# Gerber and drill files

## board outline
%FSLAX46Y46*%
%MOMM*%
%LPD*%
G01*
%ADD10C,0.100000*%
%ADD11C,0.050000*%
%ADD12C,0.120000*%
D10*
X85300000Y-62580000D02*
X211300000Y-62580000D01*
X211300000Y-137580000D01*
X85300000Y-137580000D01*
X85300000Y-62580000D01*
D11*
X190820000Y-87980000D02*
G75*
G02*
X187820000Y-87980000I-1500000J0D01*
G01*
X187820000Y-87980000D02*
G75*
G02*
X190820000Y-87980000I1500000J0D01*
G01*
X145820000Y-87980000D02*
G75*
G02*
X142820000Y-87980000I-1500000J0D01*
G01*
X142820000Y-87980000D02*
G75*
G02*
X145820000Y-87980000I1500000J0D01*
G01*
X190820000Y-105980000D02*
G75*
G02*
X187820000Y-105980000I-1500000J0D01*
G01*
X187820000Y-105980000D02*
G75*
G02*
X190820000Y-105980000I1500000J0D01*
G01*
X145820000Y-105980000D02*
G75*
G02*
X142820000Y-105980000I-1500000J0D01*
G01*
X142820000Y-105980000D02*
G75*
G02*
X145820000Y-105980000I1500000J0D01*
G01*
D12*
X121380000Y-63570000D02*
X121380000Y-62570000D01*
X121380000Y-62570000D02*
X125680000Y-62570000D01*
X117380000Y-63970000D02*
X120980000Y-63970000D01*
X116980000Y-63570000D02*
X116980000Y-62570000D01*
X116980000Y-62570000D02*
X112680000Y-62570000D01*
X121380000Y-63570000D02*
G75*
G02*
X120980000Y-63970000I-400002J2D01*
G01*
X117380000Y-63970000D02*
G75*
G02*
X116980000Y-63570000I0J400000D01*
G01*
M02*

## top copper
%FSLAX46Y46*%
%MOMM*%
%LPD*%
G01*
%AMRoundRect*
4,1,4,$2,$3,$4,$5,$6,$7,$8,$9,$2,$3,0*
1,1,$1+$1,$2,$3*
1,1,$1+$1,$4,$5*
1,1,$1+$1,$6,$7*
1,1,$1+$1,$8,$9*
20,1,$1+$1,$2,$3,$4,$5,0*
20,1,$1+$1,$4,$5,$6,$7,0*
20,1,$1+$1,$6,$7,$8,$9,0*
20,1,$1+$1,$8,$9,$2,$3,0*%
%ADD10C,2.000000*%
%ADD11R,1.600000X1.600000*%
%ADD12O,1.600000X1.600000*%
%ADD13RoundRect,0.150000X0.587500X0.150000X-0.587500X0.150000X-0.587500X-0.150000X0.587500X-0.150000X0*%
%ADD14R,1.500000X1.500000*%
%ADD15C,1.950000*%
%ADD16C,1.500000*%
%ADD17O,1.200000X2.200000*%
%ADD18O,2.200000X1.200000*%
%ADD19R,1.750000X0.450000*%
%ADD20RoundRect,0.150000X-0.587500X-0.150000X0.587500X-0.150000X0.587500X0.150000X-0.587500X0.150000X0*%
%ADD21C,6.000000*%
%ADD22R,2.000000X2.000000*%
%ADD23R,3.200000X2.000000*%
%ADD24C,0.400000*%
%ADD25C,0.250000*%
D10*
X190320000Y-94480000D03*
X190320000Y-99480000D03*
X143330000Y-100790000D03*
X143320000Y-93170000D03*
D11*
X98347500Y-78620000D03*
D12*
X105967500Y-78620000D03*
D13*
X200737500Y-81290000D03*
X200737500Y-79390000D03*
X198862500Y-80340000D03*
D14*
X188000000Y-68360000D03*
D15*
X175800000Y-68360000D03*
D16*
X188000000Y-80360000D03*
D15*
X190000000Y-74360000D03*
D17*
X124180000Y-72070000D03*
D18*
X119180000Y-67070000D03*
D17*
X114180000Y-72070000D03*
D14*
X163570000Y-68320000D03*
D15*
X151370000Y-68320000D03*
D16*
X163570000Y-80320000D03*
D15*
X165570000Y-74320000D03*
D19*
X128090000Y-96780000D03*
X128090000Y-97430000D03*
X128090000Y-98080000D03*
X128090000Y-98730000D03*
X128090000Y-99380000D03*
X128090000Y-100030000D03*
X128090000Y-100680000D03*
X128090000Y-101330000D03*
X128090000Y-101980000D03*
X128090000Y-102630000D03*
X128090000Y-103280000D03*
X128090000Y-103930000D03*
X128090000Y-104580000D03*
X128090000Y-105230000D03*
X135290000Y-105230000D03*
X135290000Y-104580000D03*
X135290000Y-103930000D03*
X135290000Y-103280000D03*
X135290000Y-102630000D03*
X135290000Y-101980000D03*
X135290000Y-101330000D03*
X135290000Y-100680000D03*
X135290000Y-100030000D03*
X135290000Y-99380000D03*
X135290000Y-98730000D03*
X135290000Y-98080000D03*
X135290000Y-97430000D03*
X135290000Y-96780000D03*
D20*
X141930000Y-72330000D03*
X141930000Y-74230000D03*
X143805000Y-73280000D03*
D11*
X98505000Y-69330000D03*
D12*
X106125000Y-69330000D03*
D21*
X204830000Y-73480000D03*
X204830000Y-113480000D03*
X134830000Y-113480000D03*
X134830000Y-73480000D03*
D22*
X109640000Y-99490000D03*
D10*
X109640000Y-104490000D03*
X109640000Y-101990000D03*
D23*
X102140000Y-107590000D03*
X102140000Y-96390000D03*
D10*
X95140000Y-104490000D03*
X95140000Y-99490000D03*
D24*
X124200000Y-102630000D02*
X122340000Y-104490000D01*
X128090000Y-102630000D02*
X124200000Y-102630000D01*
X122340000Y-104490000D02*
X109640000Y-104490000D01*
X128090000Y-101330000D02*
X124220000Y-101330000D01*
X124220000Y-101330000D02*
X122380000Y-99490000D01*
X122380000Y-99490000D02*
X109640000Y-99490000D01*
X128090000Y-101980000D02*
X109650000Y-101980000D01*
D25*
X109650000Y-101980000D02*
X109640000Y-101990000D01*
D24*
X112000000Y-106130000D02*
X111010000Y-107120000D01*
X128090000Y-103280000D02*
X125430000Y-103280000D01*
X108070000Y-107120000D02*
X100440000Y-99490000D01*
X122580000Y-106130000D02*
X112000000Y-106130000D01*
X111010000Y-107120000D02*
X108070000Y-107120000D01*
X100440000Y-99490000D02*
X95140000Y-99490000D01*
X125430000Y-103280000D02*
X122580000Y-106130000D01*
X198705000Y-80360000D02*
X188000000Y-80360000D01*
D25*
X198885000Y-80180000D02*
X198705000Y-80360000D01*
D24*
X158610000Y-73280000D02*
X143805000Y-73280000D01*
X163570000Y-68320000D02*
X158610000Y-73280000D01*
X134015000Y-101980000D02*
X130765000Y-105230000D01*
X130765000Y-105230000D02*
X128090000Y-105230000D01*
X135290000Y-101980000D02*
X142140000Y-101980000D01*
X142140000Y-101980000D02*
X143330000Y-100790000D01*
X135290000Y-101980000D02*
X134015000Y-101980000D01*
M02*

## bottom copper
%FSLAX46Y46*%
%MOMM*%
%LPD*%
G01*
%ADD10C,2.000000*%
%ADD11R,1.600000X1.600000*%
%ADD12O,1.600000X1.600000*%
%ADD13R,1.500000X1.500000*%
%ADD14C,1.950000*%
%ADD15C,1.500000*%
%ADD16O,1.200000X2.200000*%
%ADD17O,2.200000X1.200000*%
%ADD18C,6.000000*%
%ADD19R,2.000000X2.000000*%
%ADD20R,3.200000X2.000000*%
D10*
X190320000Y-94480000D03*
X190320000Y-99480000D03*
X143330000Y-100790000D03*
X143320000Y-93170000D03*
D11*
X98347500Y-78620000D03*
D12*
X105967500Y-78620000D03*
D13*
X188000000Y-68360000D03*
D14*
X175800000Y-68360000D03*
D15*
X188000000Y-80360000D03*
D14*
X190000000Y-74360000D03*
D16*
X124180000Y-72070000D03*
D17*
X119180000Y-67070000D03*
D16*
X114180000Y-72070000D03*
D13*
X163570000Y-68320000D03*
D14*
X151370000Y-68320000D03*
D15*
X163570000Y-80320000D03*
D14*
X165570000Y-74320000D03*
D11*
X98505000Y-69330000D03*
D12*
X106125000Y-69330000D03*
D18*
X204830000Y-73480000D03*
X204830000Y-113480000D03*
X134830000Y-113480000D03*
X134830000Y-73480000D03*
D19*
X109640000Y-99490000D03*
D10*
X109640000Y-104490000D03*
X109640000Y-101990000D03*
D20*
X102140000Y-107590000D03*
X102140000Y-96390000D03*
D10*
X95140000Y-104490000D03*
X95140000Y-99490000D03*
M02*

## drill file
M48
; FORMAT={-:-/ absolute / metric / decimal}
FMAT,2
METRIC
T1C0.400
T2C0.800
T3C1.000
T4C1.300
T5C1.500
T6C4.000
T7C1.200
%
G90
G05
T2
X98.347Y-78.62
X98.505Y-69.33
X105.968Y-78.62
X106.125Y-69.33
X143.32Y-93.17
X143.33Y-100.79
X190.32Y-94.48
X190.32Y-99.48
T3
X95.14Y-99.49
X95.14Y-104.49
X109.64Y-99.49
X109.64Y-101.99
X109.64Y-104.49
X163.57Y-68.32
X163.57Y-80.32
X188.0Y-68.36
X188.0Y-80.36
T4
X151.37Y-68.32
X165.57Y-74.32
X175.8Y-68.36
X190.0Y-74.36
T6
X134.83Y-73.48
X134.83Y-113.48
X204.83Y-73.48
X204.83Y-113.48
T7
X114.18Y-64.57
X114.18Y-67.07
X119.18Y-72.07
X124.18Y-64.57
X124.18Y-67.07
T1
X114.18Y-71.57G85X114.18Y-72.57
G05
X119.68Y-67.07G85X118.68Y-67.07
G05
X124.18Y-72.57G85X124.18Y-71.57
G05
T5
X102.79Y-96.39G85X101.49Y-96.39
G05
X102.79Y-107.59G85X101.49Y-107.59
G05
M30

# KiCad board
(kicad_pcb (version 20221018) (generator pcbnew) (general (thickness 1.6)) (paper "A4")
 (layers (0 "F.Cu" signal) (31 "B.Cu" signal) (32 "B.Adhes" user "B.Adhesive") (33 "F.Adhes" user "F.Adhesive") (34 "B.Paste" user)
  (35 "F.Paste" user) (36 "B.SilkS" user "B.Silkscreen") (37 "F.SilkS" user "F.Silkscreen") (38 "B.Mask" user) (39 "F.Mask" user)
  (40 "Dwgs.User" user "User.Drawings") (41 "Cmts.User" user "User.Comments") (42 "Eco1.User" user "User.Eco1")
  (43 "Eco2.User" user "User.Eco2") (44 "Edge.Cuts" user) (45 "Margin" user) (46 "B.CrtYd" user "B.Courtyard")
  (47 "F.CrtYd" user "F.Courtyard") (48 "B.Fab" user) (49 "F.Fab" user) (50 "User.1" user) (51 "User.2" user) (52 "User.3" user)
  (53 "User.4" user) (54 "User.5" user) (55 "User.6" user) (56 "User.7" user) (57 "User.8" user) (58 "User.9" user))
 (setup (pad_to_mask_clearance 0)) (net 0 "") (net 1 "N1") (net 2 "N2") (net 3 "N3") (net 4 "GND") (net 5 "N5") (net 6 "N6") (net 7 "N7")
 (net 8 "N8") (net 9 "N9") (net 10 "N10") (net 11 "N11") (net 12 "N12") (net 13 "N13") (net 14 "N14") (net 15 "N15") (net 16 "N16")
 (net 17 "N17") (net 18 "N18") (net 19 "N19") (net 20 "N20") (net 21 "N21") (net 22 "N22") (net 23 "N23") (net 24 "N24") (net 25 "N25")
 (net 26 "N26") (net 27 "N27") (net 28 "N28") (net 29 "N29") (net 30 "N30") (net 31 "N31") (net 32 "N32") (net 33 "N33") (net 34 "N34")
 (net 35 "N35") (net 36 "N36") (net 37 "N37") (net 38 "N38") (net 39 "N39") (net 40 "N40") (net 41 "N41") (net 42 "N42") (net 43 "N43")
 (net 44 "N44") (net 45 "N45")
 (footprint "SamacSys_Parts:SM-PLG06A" (layer "F.Cu") (at 190.32 96.98 -90)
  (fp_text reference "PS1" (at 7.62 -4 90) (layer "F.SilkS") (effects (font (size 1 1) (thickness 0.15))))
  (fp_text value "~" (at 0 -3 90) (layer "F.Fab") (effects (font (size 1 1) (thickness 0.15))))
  (fp_circle (center -9 1) (end -7.5 1) (stroke (width 0.05) (type default)) (fill none) (layer "Edge.Cuts"))
  (fp_circle (center -9 46) (end -7.5 46) (stroke (width 0.05) (type default)) (fill none) (layer "Edge.Cuts"))
  (fp_circle (center 9 1) (end 10.5 1) (stroke (width 0.05) (type default)) (fill none) (layer "Edge.Cuts"))
  (fp_circle (center 9 46) (end 10.5 46) (stroke (width 0.05) (type default)) (fill none) (layer "Edge.Cuts"))
  (pad "1" thru_hole circle (at -2.5 0 270) (size 2 2) (drill 0.8) (layers "*.Cu" "*.Mask") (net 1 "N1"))
  (pad "2" thru_hole circle (at 2.5 0 270) (size 2 2) (drill 0.8) (layers "*.Cu" "*.Mask") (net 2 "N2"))
  (pad "3" thru_hole circle (at 3.81 46.99 270) (size 2 2) (drill 0.8) (layers "*.Cu" "*.Mask") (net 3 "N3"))
  (pad "4" thru_hole circle (at -3.81 47 270) (size 2 2) (drill 0.8) (layers "*.Cu" "*.Mask") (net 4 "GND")))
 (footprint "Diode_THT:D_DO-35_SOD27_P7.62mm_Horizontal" (layer "F.Cu") (at 98.3475 78.62)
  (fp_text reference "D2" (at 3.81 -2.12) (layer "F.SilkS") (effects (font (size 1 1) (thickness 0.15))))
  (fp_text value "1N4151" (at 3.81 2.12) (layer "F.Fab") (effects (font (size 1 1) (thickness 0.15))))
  (pad "1" thru_hole rect (at 0 0) (size 1.6 1.6) (drill 0.8) (layers "*.Cu" "*.Mask") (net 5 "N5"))
  (pad "2" thru_hole oval (at 7.62 0) (size 1.6 1.6) (drill 0.8) (layers "*.Cu" "*.Mask") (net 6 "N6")))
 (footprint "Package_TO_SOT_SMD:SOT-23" (layer "F.Cu") (at 199.8 80.34 180)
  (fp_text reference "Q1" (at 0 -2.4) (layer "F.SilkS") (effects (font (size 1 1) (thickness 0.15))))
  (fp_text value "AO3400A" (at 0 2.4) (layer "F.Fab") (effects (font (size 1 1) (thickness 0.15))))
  (pad "1" smd roundrect (at -0.9375 -0.95 180) (size 1.475 0.6) (layers "F.Cu" "F.Paste" "F.Mask") (roundrect_rratio 0.25) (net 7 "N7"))
  (pad "2" smd roundrect (at -0.9375 0.95 180) (size 1.475 0.6) (layers "F.Cu" "F.Paste" "F.Mask") (roundrect_rratio 0.25) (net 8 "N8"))
  (pad "3" smd roundrect (at 0.9375 0 180) (size 1.475 0.6) (layers "F.Cu" "F.Paste" "F.Mask") (roundrect_rratio 0.25) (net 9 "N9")))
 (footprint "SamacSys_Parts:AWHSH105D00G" (layer "F.Cu") (at 188 68.36 180)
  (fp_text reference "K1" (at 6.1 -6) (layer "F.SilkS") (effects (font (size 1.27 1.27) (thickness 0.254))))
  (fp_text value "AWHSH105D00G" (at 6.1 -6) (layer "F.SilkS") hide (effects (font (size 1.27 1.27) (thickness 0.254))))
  (pad "1" thru_hole rect (at 0 0 180) (size 1.5 1.5) (drill 1) (layers "*.Cu" "*.Mask") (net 4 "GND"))
  (pad "2" thru_hole circle (at 12.2 0 180) (size 1.95 1.95) (drill 1.3) (layers "*.Cu" "*.Mask") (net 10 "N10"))
  (pad "3" thru_hole circle (at 0 -12 180) (size 1.5 1.5) (drill 1) (layers "*.Cu" "*.Mask") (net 9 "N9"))
  (pad "4" thru_hole circle (at -2 -6 180) (size 1.95 1.95) (drill 1.3) (layers "*.Cu" "*.Mask") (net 2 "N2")))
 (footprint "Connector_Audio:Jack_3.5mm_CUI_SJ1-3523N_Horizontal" (layer "F.Cu") (at 119.18 67.07 180)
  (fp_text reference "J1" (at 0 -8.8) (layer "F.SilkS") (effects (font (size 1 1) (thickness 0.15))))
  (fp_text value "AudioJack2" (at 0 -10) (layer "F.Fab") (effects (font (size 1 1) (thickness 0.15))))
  (fp_line (start -2.2 3.5) (end -2.2 4.5) (stroke (width 0.12) (type solid)) (layer "Edge.Cuts"))
  (fp_line (start -2.2 4.5) (end -6.5 4.5) (stroke (width 0.12) (type solid)) (layer "Edge.Cuts"))
  (fp_line (start 1.8 3.1) (end -1.8 3.1) (stroke (width 0.12) (type solid)) (layer "Edge.Cuts"))
  (fp_line (start 2.2 3.5) (end 2.2 4.5) (stroke (width 0.12) (type solid)) (layer "Edge.Cuts"))
  (fp_line (start 2.2 4.5) (end 6.5 4.5) (stroke (width 0.12) (type solid)) (layer "Edge.Cuts"))
  (fp_arc (start -2.2 3.5) (mid -2.082842 3.217158) (end -1.8 3.1) (stroke (width 0.12) (type solid)) (layer "Edge.Cuts"))
  (fp_arc (start 1.8 3.1) (mid 2.082843 3.217157) (end 2.2 3.5) (stroke (width 0.12) (type solid)) (layer "Edge.Cuts"))
  (pad "" np_thru_hole circle (at -5 0 180) (size 1.2 1.2) (drill 1.2) (layers "*.Cu"))
  (pad "" np_thru_hole circle (at -5 2.5 180) (size 1.2 1.2) (drill 1.2) (layers "*.Cu"))
  (pad "" np_thru_hole circle (at 0 -5 180) (size 1.2 1.2) (drill 1.2) (layers "*.Cu"))
  (pad "" np_thru_hole circle (at 5 0 180) (size 1.2 1.2) (drill 1.2) (layers "*.Cu"))
  (pad "" np_thru_hole circle (at 5 2.5 180) (size 1.2 1.2) (drill 1.2) (layers "*.Cu"))
  (pad "R" thru_hole oval (at -5 -5 180) (size 1.2 2.2) (drill oval 0.4 1.4) (layers "*.Cu" "*.Mask") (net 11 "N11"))
  (pad "S" thru_hole oval (at 0 0 180) (size 2.2 1.2) (drill oval 1.4 0.4) (layers "*.Cu" "*.Mask") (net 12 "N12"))
  (pad "T" thru_hole oval (at 5 -5) (size 1.2 2.2) (drill oval 0.4 1.4) (layers "*.Cu" "*.Mask") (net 4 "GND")))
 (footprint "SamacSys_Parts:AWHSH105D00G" (layer "F.Cu") (at 163.57 68.32 180)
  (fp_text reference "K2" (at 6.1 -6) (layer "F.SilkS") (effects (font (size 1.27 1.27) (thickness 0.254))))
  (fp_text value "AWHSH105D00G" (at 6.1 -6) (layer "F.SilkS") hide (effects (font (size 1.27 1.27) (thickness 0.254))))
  (pad "1" thru_hole rect (at 0 0 180) (size 1.5 1.5) (drill 1) (layers "*.Cu" "*.Mask") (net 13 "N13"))
  (pad "2" thru_hole circle (at 12.2 0 180) (size 1.95 1.95) (drill 1.3) (layers "*.Cu" "*.Mask") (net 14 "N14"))
  (pad "3" thru_hole circle (at 0 -12 180) (size 1.5 1.5) (drill 1) (layers "*.Cu" "*.Mask") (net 4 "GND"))
  (pad "4" thru_hole circle (at -2 -6 180) (size 1.95 1.95) (drill 1.3) (layers "*.Cu" "*.Mask") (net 2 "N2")))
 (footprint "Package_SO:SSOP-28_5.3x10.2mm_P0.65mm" (layer "F.Cu") (at 131.69 101.005)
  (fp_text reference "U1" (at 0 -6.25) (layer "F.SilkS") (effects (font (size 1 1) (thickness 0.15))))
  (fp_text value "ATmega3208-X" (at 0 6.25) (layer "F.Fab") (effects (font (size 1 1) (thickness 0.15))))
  (pad "1" smd rect (at -3.6 -4.225) (size 1.75 0.45) (layers "F.Cu" "F.Paste" "F.Mask") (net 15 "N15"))
  (pad "2" smd rect (at -3.6 -3.575) (size 1.75 0.45) (layers "F.Cu" "F.Paste" "F.Mask") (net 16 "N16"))
  (pad "3" smd rect (at -3.6 -2.925) (size 1.75 0.45) (layers "F.Cu" "F.Paste" "F.Mask") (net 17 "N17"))
  (pad "4" smd rect (at -3.6 -2.275) (size 1.75 0.45) (layers "F.Cu" "F.Paste" "F.Mask") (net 11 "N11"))
  (pad "5" smd rect (at -3.6 -1.625) (size 1.75 0.45) (layers "F.Cu" "F.Paste" "F.Mask") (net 12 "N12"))
  (pad "6" smd rect (at -3.6 -0.975) (size 1.75 0.45) (layers "F.Cu" "F.Paste" "F.Mask") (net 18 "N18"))
  (pad "7" smd rect (at -3.6 -0.325) (size 1.75 0.45) (layers "F.Cu" "F.Paste" "F.Mask") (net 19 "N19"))
  (pad "8" smd rect (at -3.6 0.325) (size 1.75 0.45) (layers "F.Cu" "F.Paste" "F.Mask") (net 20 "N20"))
  (pad "9" smd rect (at -3.6 0.975) (size 1.75 0.45) (layers "F.Cu" "F.Paste" "F.Mask") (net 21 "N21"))
  (pad "10" smd rect (at -3.6 1.625) (size 1.75 0.45) (layers "F.Cu" "F.Paste" "F.Mask") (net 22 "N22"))
  (pad "11" smd rect (at -3.6 2.275) (size 1.75 0.45) (layers "F.Cu" "F.Paste" "F.Mask") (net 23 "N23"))
  (pad "12" smd rect (at -3.6 2.925) (size 1.75 0.45) (layers "F.Cu" "F.Paste" "F.Mask") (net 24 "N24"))
  (pad "13" smd rect (at -3.6 3.575) (size 1.75 0.45) (layers "F.Cu" "F.Paste" "F.Mask") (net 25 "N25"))
  (pad "14" smd rect (at -3.6 4.225) (size 1.75 0.45) (layers "F.Cu" "F.Paste" "F.Mask") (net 3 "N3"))
  (pad "15" smd rect (at 3.6 4.225) (size 1.75 0.45) (layers "F.Cu" "F.Paste" "F.Mask") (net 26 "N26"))
  (pad "16" smd rect (at 3.6 3.575) (size 1.75 0.45) (layers "F.Cu" "F.Paste" "F.Mask") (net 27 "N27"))
  (pad "17" smd rect (at 3.6 2.925) (size 1.75 0.45) (layers "F.Cu" "F.Paste" "F.Mask") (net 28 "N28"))
  (pad "18" smd rect (at 3.6 2.275) (size 1.75 0.45) (layers "F.Cu" "F.Paste" "F.Mask") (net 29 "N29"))
  (pad "19" smd rect (at 3.6 1.625) (size 1.75 0.45) (layers "F.Cu" "F.Paste" "F.Mask") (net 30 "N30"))
  (pad "20" smd rect (at 3.6 0.975) (size 1.75 0.45) (layers "F.Cu" "F.Paste" "F.Mask") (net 3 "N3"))
  (pad "21" smd rect (at 3.6 0.325) (size 1.75 0.45) (layers "F.Cu" "F.Paste" "F.Mask") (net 26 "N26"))
  (pad "22" smd rect (at 3.6 -0.325) (size 1.75 0.45) (layers "F.Cu" "F.Paste" "F.Mask") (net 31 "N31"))
  (pad "23" smd rect (at 3.6 -0.975) (size 1.75 0.45) (layers "F.Cu" "F.Paste" "F.Mask") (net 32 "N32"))
  (pad "24" smd rect (at 3.6 -1.625) (size 1.75 0.45) (layers "F.Cu" "F.Paste" "F.Mask") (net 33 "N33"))
  (pad "25" smd rect (at 3.6 -2.275) (size 1.75 0.45) (layers "F.Cu" "F.Paste" "F.Mask") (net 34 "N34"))
  (pad "26" smd rect (at 3.6 -2.925) (size 1.75 0.45) (layers "F.Cu" "F.Paste" "F.Mask") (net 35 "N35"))
  (pad "27" smd rect (at 3.6 -3.575) (size 1.75 0.45) (layers "F.Cu" "F.Paste" "F.Mask") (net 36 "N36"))
  (pad "28" smd rect (at 3.6 -4.225) (size 1.75 0.45) (layers "F.Cu" "F.Paste" "F.Mask") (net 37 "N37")))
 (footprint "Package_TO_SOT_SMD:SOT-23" (layer "F.Cu") (at 142.8675 73.28)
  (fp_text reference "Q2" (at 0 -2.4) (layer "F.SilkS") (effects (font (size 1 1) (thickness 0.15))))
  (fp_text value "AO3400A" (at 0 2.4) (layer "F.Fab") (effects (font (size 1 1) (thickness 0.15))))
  (pad "1" smd roundrect (at -0.9375 -0.95) (size 1.475 0.6) (layers "F.Cu" "F.Paste" "F.Mask") (roundrect_rratio 0.25) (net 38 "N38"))
  (pad "2" smd roundrect (at -0.9375 0.95) (size 1.475 0.6) (layers "F.Cu" "F.Paste" "F.Mask") (roundrect_rratio 0.25) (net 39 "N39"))
  (pad "3" smd roundrect (at 0.9375 0) (size 1.475 0.6) (layers "F.Cu" "F.Paste" "F.Mask") (roundrect_rratio 0.25) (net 13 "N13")))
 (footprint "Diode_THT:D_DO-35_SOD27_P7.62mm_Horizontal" (layer "F.Cu") (at 98.505 69.33)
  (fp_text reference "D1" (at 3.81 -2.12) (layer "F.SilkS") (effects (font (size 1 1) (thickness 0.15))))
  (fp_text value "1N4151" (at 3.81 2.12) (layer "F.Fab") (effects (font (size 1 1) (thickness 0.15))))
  (pad "1" thru_hole rect (at 0 0) (size 1.6 1.6) (drill 0.8) (layers "*.Cu" "*.Mask") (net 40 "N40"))
  (pad "2" thru_hole oval (at 7.62 0) (size 1.6 1.6) (drill 0.8) (layers "*.Cu" "*.Mask") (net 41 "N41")))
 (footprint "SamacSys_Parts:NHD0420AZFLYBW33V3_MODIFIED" (layer "B.Cu") (at 198.33 72.48 180)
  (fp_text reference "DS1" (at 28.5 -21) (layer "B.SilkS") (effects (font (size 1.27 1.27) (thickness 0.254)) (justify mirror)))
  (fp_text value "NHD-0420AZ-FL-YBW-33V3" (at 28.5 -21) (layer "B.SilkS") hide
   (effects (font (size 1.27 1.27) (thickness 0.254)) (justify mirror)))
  (pad "MH1" thru_hole circle (at -6.5 -1 180) (size 6 6) (drill 4) (layers "*.Cu" "*.Mask") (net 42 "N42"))
  (pad "MH2" thru_hole circle (at -6.5 -41 180) (size 6 6) (drill 4) (layers "*.Cu" "*.Mask") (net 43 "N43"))
  (pad "MH3" thru_hole circle (at 63.5 -41 180) (size 6 6) (drill 4) (layers "*.Cu" "*.Mask") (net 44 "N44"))
  (pad "MH4" thru_hole circle (at 63.5 -1 180) (size 6 6) (drill 4) (layers "*.Cu" "*.Mask") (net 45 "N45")))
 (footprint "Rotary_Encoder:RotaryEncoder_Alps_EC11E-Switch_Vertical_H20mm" (layer "B.Cu") (at 109.64 99.49 180)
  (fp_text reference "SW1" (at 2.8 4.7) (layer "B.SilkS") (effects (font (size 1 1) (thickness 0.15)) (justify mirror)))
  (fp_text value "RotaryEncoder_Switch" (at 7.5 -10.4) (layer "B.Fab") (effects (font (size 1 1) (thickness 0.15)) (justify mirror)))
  (pad "A" thru_hole rect (at 0 0 180) (size 2 2) (drill 1) (layers "*.Cu" "*.Mask") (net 20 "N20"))
  (pad "B" thru_hole circle (at 0 -5 180) (size 2 2) (drill 1) (layers "*.Cu" "*.Mask") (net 22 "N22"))
  (pad "C" thru_hole circle (at 0 -2.5 180) (size 2 2) (drill 1) (layers "*.Cu" "*.Mask") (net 21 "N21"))
  (pad "MP" thru_hole rect (at 7.5 -8.1 180) (size 3.2 2) (drill oval 2.8 1.5) (layers "*.Cu" "*.Mask"))
  (pad "MP" thru_hole rect (at 7.5 3.1 180) (size 3.2 2) (drill oval 2.8 1.5) (layers "*.Cu" "*.Mask"))
  (pad "S1" thru_hole circle (at 14.5 -5 180) (size 2 2) (drill 1) (layers "*.Cu" "*.Mask") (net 4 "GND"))
  (pad "S2" thru_hole circle (at 14.5 0 180) (size 2 2) (drill 1) (layers "*.Cu" "*.Mask") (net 23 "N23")))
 (gr_rect (start 85.3 62.58) (end 211.3 137.58) (stroke (width 0.1) (type default)) (fill none) (layer "Edge.Cuts"))
 (segment (start 124.2 102.63) (end 122.34 104.49) (width 0.4) (layer "F.Cu") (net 22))
 (segment (start 128.09 102.63) (end 124.2 102.63) (width 0.4) (layer "F.Cu") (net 22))
 (segment (start 122.34 104.49) (end 109.64 104.49) (width 0.4) (layer "F.Cu") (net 22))
 (segment (start 128.09 101.33) (end 124.22 101.33) (width 0.4) (layer "F.Cu") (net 20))
 (segment (start 124.22 101.33) (end 122.38 99.49) (width 0.4) (layer "F.Cu") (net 20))
 (segment (start 122.38 99.49) (end 109.64 99.49) (width 0.4) (layer "F.Cu") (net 20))
 (segment (start 128.09 101.98) (end 109.65 101.98) (width 0.4) (layer "F.Cu") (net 21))
 (segment (start 109.65 101.98) (end 109.64 101.99) (width 0.25) (layer "F.Cu") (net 21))
 (segment (start 112 106.13) (end 111.01 107.12) (width 0.4) (layer "F.Cu") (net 23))
 (segment (start 128.09 103.28) (end 125.43 103.28) (width 0.4) (layer "F.Cu") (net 23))
 (segment (start 108.07 107.12) (end 100.44 99.49) (width 0.4) (layer "F.Cu") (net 23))
 (segment (start 122.58 106.13) (end 112 106.13) (width 0.4) (layer "F.Cu") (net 23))
 (segment (start 111.01 107.12) (end 108.07 107.12) (width 0.4) (layer "F.Cu") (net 23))
 (segment (start 100.44 99.49) (end 95.14 99.49) (width 0.4) (layer "F.Cu") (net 23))
 (segment (start 125.43 103.28) (end 122.58 106.13) (width 0.4) (layer "F.Cu") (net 23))
 (segment (start 198.705 80.36) (end 188 80.36) (width 0.4) (layer "F.Cu") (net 9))
 (segment (start 198.885 80.18) (end 198.705 80.36) (width 0.25) (layer "F.Cu") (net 9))
 (segment (start 158.61 73.28) (end 143.805 73.28) (width 0.4) (layer "F.Cu") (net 13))
 (segment (start 163.57 68.32) (end 158.61 73.28) (width 0.4) (layer "F.Cu") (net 13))
 (segment (start 134.015 101.98) (end 130.765 105.23) (width 0.4) (layer "F.Cu") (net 3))
 (segment (start 130.765 105.23) (end 128.09 105.23) (width 0.4) (layer "F.Cu") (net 3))
 (segment (start 135.29 101.98) (end 142.14 101.98) (width 0.4) (layer "F.Cu") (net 3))
 (segment (start 142.14 101.98) (end 143.33 100.79) (width 0.4) (layer "F.Cu") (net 3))
 (segment (start 135.29 101.98) (end 134.015 101.98) (width 0.4) (layer "F.Cu") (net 3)))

